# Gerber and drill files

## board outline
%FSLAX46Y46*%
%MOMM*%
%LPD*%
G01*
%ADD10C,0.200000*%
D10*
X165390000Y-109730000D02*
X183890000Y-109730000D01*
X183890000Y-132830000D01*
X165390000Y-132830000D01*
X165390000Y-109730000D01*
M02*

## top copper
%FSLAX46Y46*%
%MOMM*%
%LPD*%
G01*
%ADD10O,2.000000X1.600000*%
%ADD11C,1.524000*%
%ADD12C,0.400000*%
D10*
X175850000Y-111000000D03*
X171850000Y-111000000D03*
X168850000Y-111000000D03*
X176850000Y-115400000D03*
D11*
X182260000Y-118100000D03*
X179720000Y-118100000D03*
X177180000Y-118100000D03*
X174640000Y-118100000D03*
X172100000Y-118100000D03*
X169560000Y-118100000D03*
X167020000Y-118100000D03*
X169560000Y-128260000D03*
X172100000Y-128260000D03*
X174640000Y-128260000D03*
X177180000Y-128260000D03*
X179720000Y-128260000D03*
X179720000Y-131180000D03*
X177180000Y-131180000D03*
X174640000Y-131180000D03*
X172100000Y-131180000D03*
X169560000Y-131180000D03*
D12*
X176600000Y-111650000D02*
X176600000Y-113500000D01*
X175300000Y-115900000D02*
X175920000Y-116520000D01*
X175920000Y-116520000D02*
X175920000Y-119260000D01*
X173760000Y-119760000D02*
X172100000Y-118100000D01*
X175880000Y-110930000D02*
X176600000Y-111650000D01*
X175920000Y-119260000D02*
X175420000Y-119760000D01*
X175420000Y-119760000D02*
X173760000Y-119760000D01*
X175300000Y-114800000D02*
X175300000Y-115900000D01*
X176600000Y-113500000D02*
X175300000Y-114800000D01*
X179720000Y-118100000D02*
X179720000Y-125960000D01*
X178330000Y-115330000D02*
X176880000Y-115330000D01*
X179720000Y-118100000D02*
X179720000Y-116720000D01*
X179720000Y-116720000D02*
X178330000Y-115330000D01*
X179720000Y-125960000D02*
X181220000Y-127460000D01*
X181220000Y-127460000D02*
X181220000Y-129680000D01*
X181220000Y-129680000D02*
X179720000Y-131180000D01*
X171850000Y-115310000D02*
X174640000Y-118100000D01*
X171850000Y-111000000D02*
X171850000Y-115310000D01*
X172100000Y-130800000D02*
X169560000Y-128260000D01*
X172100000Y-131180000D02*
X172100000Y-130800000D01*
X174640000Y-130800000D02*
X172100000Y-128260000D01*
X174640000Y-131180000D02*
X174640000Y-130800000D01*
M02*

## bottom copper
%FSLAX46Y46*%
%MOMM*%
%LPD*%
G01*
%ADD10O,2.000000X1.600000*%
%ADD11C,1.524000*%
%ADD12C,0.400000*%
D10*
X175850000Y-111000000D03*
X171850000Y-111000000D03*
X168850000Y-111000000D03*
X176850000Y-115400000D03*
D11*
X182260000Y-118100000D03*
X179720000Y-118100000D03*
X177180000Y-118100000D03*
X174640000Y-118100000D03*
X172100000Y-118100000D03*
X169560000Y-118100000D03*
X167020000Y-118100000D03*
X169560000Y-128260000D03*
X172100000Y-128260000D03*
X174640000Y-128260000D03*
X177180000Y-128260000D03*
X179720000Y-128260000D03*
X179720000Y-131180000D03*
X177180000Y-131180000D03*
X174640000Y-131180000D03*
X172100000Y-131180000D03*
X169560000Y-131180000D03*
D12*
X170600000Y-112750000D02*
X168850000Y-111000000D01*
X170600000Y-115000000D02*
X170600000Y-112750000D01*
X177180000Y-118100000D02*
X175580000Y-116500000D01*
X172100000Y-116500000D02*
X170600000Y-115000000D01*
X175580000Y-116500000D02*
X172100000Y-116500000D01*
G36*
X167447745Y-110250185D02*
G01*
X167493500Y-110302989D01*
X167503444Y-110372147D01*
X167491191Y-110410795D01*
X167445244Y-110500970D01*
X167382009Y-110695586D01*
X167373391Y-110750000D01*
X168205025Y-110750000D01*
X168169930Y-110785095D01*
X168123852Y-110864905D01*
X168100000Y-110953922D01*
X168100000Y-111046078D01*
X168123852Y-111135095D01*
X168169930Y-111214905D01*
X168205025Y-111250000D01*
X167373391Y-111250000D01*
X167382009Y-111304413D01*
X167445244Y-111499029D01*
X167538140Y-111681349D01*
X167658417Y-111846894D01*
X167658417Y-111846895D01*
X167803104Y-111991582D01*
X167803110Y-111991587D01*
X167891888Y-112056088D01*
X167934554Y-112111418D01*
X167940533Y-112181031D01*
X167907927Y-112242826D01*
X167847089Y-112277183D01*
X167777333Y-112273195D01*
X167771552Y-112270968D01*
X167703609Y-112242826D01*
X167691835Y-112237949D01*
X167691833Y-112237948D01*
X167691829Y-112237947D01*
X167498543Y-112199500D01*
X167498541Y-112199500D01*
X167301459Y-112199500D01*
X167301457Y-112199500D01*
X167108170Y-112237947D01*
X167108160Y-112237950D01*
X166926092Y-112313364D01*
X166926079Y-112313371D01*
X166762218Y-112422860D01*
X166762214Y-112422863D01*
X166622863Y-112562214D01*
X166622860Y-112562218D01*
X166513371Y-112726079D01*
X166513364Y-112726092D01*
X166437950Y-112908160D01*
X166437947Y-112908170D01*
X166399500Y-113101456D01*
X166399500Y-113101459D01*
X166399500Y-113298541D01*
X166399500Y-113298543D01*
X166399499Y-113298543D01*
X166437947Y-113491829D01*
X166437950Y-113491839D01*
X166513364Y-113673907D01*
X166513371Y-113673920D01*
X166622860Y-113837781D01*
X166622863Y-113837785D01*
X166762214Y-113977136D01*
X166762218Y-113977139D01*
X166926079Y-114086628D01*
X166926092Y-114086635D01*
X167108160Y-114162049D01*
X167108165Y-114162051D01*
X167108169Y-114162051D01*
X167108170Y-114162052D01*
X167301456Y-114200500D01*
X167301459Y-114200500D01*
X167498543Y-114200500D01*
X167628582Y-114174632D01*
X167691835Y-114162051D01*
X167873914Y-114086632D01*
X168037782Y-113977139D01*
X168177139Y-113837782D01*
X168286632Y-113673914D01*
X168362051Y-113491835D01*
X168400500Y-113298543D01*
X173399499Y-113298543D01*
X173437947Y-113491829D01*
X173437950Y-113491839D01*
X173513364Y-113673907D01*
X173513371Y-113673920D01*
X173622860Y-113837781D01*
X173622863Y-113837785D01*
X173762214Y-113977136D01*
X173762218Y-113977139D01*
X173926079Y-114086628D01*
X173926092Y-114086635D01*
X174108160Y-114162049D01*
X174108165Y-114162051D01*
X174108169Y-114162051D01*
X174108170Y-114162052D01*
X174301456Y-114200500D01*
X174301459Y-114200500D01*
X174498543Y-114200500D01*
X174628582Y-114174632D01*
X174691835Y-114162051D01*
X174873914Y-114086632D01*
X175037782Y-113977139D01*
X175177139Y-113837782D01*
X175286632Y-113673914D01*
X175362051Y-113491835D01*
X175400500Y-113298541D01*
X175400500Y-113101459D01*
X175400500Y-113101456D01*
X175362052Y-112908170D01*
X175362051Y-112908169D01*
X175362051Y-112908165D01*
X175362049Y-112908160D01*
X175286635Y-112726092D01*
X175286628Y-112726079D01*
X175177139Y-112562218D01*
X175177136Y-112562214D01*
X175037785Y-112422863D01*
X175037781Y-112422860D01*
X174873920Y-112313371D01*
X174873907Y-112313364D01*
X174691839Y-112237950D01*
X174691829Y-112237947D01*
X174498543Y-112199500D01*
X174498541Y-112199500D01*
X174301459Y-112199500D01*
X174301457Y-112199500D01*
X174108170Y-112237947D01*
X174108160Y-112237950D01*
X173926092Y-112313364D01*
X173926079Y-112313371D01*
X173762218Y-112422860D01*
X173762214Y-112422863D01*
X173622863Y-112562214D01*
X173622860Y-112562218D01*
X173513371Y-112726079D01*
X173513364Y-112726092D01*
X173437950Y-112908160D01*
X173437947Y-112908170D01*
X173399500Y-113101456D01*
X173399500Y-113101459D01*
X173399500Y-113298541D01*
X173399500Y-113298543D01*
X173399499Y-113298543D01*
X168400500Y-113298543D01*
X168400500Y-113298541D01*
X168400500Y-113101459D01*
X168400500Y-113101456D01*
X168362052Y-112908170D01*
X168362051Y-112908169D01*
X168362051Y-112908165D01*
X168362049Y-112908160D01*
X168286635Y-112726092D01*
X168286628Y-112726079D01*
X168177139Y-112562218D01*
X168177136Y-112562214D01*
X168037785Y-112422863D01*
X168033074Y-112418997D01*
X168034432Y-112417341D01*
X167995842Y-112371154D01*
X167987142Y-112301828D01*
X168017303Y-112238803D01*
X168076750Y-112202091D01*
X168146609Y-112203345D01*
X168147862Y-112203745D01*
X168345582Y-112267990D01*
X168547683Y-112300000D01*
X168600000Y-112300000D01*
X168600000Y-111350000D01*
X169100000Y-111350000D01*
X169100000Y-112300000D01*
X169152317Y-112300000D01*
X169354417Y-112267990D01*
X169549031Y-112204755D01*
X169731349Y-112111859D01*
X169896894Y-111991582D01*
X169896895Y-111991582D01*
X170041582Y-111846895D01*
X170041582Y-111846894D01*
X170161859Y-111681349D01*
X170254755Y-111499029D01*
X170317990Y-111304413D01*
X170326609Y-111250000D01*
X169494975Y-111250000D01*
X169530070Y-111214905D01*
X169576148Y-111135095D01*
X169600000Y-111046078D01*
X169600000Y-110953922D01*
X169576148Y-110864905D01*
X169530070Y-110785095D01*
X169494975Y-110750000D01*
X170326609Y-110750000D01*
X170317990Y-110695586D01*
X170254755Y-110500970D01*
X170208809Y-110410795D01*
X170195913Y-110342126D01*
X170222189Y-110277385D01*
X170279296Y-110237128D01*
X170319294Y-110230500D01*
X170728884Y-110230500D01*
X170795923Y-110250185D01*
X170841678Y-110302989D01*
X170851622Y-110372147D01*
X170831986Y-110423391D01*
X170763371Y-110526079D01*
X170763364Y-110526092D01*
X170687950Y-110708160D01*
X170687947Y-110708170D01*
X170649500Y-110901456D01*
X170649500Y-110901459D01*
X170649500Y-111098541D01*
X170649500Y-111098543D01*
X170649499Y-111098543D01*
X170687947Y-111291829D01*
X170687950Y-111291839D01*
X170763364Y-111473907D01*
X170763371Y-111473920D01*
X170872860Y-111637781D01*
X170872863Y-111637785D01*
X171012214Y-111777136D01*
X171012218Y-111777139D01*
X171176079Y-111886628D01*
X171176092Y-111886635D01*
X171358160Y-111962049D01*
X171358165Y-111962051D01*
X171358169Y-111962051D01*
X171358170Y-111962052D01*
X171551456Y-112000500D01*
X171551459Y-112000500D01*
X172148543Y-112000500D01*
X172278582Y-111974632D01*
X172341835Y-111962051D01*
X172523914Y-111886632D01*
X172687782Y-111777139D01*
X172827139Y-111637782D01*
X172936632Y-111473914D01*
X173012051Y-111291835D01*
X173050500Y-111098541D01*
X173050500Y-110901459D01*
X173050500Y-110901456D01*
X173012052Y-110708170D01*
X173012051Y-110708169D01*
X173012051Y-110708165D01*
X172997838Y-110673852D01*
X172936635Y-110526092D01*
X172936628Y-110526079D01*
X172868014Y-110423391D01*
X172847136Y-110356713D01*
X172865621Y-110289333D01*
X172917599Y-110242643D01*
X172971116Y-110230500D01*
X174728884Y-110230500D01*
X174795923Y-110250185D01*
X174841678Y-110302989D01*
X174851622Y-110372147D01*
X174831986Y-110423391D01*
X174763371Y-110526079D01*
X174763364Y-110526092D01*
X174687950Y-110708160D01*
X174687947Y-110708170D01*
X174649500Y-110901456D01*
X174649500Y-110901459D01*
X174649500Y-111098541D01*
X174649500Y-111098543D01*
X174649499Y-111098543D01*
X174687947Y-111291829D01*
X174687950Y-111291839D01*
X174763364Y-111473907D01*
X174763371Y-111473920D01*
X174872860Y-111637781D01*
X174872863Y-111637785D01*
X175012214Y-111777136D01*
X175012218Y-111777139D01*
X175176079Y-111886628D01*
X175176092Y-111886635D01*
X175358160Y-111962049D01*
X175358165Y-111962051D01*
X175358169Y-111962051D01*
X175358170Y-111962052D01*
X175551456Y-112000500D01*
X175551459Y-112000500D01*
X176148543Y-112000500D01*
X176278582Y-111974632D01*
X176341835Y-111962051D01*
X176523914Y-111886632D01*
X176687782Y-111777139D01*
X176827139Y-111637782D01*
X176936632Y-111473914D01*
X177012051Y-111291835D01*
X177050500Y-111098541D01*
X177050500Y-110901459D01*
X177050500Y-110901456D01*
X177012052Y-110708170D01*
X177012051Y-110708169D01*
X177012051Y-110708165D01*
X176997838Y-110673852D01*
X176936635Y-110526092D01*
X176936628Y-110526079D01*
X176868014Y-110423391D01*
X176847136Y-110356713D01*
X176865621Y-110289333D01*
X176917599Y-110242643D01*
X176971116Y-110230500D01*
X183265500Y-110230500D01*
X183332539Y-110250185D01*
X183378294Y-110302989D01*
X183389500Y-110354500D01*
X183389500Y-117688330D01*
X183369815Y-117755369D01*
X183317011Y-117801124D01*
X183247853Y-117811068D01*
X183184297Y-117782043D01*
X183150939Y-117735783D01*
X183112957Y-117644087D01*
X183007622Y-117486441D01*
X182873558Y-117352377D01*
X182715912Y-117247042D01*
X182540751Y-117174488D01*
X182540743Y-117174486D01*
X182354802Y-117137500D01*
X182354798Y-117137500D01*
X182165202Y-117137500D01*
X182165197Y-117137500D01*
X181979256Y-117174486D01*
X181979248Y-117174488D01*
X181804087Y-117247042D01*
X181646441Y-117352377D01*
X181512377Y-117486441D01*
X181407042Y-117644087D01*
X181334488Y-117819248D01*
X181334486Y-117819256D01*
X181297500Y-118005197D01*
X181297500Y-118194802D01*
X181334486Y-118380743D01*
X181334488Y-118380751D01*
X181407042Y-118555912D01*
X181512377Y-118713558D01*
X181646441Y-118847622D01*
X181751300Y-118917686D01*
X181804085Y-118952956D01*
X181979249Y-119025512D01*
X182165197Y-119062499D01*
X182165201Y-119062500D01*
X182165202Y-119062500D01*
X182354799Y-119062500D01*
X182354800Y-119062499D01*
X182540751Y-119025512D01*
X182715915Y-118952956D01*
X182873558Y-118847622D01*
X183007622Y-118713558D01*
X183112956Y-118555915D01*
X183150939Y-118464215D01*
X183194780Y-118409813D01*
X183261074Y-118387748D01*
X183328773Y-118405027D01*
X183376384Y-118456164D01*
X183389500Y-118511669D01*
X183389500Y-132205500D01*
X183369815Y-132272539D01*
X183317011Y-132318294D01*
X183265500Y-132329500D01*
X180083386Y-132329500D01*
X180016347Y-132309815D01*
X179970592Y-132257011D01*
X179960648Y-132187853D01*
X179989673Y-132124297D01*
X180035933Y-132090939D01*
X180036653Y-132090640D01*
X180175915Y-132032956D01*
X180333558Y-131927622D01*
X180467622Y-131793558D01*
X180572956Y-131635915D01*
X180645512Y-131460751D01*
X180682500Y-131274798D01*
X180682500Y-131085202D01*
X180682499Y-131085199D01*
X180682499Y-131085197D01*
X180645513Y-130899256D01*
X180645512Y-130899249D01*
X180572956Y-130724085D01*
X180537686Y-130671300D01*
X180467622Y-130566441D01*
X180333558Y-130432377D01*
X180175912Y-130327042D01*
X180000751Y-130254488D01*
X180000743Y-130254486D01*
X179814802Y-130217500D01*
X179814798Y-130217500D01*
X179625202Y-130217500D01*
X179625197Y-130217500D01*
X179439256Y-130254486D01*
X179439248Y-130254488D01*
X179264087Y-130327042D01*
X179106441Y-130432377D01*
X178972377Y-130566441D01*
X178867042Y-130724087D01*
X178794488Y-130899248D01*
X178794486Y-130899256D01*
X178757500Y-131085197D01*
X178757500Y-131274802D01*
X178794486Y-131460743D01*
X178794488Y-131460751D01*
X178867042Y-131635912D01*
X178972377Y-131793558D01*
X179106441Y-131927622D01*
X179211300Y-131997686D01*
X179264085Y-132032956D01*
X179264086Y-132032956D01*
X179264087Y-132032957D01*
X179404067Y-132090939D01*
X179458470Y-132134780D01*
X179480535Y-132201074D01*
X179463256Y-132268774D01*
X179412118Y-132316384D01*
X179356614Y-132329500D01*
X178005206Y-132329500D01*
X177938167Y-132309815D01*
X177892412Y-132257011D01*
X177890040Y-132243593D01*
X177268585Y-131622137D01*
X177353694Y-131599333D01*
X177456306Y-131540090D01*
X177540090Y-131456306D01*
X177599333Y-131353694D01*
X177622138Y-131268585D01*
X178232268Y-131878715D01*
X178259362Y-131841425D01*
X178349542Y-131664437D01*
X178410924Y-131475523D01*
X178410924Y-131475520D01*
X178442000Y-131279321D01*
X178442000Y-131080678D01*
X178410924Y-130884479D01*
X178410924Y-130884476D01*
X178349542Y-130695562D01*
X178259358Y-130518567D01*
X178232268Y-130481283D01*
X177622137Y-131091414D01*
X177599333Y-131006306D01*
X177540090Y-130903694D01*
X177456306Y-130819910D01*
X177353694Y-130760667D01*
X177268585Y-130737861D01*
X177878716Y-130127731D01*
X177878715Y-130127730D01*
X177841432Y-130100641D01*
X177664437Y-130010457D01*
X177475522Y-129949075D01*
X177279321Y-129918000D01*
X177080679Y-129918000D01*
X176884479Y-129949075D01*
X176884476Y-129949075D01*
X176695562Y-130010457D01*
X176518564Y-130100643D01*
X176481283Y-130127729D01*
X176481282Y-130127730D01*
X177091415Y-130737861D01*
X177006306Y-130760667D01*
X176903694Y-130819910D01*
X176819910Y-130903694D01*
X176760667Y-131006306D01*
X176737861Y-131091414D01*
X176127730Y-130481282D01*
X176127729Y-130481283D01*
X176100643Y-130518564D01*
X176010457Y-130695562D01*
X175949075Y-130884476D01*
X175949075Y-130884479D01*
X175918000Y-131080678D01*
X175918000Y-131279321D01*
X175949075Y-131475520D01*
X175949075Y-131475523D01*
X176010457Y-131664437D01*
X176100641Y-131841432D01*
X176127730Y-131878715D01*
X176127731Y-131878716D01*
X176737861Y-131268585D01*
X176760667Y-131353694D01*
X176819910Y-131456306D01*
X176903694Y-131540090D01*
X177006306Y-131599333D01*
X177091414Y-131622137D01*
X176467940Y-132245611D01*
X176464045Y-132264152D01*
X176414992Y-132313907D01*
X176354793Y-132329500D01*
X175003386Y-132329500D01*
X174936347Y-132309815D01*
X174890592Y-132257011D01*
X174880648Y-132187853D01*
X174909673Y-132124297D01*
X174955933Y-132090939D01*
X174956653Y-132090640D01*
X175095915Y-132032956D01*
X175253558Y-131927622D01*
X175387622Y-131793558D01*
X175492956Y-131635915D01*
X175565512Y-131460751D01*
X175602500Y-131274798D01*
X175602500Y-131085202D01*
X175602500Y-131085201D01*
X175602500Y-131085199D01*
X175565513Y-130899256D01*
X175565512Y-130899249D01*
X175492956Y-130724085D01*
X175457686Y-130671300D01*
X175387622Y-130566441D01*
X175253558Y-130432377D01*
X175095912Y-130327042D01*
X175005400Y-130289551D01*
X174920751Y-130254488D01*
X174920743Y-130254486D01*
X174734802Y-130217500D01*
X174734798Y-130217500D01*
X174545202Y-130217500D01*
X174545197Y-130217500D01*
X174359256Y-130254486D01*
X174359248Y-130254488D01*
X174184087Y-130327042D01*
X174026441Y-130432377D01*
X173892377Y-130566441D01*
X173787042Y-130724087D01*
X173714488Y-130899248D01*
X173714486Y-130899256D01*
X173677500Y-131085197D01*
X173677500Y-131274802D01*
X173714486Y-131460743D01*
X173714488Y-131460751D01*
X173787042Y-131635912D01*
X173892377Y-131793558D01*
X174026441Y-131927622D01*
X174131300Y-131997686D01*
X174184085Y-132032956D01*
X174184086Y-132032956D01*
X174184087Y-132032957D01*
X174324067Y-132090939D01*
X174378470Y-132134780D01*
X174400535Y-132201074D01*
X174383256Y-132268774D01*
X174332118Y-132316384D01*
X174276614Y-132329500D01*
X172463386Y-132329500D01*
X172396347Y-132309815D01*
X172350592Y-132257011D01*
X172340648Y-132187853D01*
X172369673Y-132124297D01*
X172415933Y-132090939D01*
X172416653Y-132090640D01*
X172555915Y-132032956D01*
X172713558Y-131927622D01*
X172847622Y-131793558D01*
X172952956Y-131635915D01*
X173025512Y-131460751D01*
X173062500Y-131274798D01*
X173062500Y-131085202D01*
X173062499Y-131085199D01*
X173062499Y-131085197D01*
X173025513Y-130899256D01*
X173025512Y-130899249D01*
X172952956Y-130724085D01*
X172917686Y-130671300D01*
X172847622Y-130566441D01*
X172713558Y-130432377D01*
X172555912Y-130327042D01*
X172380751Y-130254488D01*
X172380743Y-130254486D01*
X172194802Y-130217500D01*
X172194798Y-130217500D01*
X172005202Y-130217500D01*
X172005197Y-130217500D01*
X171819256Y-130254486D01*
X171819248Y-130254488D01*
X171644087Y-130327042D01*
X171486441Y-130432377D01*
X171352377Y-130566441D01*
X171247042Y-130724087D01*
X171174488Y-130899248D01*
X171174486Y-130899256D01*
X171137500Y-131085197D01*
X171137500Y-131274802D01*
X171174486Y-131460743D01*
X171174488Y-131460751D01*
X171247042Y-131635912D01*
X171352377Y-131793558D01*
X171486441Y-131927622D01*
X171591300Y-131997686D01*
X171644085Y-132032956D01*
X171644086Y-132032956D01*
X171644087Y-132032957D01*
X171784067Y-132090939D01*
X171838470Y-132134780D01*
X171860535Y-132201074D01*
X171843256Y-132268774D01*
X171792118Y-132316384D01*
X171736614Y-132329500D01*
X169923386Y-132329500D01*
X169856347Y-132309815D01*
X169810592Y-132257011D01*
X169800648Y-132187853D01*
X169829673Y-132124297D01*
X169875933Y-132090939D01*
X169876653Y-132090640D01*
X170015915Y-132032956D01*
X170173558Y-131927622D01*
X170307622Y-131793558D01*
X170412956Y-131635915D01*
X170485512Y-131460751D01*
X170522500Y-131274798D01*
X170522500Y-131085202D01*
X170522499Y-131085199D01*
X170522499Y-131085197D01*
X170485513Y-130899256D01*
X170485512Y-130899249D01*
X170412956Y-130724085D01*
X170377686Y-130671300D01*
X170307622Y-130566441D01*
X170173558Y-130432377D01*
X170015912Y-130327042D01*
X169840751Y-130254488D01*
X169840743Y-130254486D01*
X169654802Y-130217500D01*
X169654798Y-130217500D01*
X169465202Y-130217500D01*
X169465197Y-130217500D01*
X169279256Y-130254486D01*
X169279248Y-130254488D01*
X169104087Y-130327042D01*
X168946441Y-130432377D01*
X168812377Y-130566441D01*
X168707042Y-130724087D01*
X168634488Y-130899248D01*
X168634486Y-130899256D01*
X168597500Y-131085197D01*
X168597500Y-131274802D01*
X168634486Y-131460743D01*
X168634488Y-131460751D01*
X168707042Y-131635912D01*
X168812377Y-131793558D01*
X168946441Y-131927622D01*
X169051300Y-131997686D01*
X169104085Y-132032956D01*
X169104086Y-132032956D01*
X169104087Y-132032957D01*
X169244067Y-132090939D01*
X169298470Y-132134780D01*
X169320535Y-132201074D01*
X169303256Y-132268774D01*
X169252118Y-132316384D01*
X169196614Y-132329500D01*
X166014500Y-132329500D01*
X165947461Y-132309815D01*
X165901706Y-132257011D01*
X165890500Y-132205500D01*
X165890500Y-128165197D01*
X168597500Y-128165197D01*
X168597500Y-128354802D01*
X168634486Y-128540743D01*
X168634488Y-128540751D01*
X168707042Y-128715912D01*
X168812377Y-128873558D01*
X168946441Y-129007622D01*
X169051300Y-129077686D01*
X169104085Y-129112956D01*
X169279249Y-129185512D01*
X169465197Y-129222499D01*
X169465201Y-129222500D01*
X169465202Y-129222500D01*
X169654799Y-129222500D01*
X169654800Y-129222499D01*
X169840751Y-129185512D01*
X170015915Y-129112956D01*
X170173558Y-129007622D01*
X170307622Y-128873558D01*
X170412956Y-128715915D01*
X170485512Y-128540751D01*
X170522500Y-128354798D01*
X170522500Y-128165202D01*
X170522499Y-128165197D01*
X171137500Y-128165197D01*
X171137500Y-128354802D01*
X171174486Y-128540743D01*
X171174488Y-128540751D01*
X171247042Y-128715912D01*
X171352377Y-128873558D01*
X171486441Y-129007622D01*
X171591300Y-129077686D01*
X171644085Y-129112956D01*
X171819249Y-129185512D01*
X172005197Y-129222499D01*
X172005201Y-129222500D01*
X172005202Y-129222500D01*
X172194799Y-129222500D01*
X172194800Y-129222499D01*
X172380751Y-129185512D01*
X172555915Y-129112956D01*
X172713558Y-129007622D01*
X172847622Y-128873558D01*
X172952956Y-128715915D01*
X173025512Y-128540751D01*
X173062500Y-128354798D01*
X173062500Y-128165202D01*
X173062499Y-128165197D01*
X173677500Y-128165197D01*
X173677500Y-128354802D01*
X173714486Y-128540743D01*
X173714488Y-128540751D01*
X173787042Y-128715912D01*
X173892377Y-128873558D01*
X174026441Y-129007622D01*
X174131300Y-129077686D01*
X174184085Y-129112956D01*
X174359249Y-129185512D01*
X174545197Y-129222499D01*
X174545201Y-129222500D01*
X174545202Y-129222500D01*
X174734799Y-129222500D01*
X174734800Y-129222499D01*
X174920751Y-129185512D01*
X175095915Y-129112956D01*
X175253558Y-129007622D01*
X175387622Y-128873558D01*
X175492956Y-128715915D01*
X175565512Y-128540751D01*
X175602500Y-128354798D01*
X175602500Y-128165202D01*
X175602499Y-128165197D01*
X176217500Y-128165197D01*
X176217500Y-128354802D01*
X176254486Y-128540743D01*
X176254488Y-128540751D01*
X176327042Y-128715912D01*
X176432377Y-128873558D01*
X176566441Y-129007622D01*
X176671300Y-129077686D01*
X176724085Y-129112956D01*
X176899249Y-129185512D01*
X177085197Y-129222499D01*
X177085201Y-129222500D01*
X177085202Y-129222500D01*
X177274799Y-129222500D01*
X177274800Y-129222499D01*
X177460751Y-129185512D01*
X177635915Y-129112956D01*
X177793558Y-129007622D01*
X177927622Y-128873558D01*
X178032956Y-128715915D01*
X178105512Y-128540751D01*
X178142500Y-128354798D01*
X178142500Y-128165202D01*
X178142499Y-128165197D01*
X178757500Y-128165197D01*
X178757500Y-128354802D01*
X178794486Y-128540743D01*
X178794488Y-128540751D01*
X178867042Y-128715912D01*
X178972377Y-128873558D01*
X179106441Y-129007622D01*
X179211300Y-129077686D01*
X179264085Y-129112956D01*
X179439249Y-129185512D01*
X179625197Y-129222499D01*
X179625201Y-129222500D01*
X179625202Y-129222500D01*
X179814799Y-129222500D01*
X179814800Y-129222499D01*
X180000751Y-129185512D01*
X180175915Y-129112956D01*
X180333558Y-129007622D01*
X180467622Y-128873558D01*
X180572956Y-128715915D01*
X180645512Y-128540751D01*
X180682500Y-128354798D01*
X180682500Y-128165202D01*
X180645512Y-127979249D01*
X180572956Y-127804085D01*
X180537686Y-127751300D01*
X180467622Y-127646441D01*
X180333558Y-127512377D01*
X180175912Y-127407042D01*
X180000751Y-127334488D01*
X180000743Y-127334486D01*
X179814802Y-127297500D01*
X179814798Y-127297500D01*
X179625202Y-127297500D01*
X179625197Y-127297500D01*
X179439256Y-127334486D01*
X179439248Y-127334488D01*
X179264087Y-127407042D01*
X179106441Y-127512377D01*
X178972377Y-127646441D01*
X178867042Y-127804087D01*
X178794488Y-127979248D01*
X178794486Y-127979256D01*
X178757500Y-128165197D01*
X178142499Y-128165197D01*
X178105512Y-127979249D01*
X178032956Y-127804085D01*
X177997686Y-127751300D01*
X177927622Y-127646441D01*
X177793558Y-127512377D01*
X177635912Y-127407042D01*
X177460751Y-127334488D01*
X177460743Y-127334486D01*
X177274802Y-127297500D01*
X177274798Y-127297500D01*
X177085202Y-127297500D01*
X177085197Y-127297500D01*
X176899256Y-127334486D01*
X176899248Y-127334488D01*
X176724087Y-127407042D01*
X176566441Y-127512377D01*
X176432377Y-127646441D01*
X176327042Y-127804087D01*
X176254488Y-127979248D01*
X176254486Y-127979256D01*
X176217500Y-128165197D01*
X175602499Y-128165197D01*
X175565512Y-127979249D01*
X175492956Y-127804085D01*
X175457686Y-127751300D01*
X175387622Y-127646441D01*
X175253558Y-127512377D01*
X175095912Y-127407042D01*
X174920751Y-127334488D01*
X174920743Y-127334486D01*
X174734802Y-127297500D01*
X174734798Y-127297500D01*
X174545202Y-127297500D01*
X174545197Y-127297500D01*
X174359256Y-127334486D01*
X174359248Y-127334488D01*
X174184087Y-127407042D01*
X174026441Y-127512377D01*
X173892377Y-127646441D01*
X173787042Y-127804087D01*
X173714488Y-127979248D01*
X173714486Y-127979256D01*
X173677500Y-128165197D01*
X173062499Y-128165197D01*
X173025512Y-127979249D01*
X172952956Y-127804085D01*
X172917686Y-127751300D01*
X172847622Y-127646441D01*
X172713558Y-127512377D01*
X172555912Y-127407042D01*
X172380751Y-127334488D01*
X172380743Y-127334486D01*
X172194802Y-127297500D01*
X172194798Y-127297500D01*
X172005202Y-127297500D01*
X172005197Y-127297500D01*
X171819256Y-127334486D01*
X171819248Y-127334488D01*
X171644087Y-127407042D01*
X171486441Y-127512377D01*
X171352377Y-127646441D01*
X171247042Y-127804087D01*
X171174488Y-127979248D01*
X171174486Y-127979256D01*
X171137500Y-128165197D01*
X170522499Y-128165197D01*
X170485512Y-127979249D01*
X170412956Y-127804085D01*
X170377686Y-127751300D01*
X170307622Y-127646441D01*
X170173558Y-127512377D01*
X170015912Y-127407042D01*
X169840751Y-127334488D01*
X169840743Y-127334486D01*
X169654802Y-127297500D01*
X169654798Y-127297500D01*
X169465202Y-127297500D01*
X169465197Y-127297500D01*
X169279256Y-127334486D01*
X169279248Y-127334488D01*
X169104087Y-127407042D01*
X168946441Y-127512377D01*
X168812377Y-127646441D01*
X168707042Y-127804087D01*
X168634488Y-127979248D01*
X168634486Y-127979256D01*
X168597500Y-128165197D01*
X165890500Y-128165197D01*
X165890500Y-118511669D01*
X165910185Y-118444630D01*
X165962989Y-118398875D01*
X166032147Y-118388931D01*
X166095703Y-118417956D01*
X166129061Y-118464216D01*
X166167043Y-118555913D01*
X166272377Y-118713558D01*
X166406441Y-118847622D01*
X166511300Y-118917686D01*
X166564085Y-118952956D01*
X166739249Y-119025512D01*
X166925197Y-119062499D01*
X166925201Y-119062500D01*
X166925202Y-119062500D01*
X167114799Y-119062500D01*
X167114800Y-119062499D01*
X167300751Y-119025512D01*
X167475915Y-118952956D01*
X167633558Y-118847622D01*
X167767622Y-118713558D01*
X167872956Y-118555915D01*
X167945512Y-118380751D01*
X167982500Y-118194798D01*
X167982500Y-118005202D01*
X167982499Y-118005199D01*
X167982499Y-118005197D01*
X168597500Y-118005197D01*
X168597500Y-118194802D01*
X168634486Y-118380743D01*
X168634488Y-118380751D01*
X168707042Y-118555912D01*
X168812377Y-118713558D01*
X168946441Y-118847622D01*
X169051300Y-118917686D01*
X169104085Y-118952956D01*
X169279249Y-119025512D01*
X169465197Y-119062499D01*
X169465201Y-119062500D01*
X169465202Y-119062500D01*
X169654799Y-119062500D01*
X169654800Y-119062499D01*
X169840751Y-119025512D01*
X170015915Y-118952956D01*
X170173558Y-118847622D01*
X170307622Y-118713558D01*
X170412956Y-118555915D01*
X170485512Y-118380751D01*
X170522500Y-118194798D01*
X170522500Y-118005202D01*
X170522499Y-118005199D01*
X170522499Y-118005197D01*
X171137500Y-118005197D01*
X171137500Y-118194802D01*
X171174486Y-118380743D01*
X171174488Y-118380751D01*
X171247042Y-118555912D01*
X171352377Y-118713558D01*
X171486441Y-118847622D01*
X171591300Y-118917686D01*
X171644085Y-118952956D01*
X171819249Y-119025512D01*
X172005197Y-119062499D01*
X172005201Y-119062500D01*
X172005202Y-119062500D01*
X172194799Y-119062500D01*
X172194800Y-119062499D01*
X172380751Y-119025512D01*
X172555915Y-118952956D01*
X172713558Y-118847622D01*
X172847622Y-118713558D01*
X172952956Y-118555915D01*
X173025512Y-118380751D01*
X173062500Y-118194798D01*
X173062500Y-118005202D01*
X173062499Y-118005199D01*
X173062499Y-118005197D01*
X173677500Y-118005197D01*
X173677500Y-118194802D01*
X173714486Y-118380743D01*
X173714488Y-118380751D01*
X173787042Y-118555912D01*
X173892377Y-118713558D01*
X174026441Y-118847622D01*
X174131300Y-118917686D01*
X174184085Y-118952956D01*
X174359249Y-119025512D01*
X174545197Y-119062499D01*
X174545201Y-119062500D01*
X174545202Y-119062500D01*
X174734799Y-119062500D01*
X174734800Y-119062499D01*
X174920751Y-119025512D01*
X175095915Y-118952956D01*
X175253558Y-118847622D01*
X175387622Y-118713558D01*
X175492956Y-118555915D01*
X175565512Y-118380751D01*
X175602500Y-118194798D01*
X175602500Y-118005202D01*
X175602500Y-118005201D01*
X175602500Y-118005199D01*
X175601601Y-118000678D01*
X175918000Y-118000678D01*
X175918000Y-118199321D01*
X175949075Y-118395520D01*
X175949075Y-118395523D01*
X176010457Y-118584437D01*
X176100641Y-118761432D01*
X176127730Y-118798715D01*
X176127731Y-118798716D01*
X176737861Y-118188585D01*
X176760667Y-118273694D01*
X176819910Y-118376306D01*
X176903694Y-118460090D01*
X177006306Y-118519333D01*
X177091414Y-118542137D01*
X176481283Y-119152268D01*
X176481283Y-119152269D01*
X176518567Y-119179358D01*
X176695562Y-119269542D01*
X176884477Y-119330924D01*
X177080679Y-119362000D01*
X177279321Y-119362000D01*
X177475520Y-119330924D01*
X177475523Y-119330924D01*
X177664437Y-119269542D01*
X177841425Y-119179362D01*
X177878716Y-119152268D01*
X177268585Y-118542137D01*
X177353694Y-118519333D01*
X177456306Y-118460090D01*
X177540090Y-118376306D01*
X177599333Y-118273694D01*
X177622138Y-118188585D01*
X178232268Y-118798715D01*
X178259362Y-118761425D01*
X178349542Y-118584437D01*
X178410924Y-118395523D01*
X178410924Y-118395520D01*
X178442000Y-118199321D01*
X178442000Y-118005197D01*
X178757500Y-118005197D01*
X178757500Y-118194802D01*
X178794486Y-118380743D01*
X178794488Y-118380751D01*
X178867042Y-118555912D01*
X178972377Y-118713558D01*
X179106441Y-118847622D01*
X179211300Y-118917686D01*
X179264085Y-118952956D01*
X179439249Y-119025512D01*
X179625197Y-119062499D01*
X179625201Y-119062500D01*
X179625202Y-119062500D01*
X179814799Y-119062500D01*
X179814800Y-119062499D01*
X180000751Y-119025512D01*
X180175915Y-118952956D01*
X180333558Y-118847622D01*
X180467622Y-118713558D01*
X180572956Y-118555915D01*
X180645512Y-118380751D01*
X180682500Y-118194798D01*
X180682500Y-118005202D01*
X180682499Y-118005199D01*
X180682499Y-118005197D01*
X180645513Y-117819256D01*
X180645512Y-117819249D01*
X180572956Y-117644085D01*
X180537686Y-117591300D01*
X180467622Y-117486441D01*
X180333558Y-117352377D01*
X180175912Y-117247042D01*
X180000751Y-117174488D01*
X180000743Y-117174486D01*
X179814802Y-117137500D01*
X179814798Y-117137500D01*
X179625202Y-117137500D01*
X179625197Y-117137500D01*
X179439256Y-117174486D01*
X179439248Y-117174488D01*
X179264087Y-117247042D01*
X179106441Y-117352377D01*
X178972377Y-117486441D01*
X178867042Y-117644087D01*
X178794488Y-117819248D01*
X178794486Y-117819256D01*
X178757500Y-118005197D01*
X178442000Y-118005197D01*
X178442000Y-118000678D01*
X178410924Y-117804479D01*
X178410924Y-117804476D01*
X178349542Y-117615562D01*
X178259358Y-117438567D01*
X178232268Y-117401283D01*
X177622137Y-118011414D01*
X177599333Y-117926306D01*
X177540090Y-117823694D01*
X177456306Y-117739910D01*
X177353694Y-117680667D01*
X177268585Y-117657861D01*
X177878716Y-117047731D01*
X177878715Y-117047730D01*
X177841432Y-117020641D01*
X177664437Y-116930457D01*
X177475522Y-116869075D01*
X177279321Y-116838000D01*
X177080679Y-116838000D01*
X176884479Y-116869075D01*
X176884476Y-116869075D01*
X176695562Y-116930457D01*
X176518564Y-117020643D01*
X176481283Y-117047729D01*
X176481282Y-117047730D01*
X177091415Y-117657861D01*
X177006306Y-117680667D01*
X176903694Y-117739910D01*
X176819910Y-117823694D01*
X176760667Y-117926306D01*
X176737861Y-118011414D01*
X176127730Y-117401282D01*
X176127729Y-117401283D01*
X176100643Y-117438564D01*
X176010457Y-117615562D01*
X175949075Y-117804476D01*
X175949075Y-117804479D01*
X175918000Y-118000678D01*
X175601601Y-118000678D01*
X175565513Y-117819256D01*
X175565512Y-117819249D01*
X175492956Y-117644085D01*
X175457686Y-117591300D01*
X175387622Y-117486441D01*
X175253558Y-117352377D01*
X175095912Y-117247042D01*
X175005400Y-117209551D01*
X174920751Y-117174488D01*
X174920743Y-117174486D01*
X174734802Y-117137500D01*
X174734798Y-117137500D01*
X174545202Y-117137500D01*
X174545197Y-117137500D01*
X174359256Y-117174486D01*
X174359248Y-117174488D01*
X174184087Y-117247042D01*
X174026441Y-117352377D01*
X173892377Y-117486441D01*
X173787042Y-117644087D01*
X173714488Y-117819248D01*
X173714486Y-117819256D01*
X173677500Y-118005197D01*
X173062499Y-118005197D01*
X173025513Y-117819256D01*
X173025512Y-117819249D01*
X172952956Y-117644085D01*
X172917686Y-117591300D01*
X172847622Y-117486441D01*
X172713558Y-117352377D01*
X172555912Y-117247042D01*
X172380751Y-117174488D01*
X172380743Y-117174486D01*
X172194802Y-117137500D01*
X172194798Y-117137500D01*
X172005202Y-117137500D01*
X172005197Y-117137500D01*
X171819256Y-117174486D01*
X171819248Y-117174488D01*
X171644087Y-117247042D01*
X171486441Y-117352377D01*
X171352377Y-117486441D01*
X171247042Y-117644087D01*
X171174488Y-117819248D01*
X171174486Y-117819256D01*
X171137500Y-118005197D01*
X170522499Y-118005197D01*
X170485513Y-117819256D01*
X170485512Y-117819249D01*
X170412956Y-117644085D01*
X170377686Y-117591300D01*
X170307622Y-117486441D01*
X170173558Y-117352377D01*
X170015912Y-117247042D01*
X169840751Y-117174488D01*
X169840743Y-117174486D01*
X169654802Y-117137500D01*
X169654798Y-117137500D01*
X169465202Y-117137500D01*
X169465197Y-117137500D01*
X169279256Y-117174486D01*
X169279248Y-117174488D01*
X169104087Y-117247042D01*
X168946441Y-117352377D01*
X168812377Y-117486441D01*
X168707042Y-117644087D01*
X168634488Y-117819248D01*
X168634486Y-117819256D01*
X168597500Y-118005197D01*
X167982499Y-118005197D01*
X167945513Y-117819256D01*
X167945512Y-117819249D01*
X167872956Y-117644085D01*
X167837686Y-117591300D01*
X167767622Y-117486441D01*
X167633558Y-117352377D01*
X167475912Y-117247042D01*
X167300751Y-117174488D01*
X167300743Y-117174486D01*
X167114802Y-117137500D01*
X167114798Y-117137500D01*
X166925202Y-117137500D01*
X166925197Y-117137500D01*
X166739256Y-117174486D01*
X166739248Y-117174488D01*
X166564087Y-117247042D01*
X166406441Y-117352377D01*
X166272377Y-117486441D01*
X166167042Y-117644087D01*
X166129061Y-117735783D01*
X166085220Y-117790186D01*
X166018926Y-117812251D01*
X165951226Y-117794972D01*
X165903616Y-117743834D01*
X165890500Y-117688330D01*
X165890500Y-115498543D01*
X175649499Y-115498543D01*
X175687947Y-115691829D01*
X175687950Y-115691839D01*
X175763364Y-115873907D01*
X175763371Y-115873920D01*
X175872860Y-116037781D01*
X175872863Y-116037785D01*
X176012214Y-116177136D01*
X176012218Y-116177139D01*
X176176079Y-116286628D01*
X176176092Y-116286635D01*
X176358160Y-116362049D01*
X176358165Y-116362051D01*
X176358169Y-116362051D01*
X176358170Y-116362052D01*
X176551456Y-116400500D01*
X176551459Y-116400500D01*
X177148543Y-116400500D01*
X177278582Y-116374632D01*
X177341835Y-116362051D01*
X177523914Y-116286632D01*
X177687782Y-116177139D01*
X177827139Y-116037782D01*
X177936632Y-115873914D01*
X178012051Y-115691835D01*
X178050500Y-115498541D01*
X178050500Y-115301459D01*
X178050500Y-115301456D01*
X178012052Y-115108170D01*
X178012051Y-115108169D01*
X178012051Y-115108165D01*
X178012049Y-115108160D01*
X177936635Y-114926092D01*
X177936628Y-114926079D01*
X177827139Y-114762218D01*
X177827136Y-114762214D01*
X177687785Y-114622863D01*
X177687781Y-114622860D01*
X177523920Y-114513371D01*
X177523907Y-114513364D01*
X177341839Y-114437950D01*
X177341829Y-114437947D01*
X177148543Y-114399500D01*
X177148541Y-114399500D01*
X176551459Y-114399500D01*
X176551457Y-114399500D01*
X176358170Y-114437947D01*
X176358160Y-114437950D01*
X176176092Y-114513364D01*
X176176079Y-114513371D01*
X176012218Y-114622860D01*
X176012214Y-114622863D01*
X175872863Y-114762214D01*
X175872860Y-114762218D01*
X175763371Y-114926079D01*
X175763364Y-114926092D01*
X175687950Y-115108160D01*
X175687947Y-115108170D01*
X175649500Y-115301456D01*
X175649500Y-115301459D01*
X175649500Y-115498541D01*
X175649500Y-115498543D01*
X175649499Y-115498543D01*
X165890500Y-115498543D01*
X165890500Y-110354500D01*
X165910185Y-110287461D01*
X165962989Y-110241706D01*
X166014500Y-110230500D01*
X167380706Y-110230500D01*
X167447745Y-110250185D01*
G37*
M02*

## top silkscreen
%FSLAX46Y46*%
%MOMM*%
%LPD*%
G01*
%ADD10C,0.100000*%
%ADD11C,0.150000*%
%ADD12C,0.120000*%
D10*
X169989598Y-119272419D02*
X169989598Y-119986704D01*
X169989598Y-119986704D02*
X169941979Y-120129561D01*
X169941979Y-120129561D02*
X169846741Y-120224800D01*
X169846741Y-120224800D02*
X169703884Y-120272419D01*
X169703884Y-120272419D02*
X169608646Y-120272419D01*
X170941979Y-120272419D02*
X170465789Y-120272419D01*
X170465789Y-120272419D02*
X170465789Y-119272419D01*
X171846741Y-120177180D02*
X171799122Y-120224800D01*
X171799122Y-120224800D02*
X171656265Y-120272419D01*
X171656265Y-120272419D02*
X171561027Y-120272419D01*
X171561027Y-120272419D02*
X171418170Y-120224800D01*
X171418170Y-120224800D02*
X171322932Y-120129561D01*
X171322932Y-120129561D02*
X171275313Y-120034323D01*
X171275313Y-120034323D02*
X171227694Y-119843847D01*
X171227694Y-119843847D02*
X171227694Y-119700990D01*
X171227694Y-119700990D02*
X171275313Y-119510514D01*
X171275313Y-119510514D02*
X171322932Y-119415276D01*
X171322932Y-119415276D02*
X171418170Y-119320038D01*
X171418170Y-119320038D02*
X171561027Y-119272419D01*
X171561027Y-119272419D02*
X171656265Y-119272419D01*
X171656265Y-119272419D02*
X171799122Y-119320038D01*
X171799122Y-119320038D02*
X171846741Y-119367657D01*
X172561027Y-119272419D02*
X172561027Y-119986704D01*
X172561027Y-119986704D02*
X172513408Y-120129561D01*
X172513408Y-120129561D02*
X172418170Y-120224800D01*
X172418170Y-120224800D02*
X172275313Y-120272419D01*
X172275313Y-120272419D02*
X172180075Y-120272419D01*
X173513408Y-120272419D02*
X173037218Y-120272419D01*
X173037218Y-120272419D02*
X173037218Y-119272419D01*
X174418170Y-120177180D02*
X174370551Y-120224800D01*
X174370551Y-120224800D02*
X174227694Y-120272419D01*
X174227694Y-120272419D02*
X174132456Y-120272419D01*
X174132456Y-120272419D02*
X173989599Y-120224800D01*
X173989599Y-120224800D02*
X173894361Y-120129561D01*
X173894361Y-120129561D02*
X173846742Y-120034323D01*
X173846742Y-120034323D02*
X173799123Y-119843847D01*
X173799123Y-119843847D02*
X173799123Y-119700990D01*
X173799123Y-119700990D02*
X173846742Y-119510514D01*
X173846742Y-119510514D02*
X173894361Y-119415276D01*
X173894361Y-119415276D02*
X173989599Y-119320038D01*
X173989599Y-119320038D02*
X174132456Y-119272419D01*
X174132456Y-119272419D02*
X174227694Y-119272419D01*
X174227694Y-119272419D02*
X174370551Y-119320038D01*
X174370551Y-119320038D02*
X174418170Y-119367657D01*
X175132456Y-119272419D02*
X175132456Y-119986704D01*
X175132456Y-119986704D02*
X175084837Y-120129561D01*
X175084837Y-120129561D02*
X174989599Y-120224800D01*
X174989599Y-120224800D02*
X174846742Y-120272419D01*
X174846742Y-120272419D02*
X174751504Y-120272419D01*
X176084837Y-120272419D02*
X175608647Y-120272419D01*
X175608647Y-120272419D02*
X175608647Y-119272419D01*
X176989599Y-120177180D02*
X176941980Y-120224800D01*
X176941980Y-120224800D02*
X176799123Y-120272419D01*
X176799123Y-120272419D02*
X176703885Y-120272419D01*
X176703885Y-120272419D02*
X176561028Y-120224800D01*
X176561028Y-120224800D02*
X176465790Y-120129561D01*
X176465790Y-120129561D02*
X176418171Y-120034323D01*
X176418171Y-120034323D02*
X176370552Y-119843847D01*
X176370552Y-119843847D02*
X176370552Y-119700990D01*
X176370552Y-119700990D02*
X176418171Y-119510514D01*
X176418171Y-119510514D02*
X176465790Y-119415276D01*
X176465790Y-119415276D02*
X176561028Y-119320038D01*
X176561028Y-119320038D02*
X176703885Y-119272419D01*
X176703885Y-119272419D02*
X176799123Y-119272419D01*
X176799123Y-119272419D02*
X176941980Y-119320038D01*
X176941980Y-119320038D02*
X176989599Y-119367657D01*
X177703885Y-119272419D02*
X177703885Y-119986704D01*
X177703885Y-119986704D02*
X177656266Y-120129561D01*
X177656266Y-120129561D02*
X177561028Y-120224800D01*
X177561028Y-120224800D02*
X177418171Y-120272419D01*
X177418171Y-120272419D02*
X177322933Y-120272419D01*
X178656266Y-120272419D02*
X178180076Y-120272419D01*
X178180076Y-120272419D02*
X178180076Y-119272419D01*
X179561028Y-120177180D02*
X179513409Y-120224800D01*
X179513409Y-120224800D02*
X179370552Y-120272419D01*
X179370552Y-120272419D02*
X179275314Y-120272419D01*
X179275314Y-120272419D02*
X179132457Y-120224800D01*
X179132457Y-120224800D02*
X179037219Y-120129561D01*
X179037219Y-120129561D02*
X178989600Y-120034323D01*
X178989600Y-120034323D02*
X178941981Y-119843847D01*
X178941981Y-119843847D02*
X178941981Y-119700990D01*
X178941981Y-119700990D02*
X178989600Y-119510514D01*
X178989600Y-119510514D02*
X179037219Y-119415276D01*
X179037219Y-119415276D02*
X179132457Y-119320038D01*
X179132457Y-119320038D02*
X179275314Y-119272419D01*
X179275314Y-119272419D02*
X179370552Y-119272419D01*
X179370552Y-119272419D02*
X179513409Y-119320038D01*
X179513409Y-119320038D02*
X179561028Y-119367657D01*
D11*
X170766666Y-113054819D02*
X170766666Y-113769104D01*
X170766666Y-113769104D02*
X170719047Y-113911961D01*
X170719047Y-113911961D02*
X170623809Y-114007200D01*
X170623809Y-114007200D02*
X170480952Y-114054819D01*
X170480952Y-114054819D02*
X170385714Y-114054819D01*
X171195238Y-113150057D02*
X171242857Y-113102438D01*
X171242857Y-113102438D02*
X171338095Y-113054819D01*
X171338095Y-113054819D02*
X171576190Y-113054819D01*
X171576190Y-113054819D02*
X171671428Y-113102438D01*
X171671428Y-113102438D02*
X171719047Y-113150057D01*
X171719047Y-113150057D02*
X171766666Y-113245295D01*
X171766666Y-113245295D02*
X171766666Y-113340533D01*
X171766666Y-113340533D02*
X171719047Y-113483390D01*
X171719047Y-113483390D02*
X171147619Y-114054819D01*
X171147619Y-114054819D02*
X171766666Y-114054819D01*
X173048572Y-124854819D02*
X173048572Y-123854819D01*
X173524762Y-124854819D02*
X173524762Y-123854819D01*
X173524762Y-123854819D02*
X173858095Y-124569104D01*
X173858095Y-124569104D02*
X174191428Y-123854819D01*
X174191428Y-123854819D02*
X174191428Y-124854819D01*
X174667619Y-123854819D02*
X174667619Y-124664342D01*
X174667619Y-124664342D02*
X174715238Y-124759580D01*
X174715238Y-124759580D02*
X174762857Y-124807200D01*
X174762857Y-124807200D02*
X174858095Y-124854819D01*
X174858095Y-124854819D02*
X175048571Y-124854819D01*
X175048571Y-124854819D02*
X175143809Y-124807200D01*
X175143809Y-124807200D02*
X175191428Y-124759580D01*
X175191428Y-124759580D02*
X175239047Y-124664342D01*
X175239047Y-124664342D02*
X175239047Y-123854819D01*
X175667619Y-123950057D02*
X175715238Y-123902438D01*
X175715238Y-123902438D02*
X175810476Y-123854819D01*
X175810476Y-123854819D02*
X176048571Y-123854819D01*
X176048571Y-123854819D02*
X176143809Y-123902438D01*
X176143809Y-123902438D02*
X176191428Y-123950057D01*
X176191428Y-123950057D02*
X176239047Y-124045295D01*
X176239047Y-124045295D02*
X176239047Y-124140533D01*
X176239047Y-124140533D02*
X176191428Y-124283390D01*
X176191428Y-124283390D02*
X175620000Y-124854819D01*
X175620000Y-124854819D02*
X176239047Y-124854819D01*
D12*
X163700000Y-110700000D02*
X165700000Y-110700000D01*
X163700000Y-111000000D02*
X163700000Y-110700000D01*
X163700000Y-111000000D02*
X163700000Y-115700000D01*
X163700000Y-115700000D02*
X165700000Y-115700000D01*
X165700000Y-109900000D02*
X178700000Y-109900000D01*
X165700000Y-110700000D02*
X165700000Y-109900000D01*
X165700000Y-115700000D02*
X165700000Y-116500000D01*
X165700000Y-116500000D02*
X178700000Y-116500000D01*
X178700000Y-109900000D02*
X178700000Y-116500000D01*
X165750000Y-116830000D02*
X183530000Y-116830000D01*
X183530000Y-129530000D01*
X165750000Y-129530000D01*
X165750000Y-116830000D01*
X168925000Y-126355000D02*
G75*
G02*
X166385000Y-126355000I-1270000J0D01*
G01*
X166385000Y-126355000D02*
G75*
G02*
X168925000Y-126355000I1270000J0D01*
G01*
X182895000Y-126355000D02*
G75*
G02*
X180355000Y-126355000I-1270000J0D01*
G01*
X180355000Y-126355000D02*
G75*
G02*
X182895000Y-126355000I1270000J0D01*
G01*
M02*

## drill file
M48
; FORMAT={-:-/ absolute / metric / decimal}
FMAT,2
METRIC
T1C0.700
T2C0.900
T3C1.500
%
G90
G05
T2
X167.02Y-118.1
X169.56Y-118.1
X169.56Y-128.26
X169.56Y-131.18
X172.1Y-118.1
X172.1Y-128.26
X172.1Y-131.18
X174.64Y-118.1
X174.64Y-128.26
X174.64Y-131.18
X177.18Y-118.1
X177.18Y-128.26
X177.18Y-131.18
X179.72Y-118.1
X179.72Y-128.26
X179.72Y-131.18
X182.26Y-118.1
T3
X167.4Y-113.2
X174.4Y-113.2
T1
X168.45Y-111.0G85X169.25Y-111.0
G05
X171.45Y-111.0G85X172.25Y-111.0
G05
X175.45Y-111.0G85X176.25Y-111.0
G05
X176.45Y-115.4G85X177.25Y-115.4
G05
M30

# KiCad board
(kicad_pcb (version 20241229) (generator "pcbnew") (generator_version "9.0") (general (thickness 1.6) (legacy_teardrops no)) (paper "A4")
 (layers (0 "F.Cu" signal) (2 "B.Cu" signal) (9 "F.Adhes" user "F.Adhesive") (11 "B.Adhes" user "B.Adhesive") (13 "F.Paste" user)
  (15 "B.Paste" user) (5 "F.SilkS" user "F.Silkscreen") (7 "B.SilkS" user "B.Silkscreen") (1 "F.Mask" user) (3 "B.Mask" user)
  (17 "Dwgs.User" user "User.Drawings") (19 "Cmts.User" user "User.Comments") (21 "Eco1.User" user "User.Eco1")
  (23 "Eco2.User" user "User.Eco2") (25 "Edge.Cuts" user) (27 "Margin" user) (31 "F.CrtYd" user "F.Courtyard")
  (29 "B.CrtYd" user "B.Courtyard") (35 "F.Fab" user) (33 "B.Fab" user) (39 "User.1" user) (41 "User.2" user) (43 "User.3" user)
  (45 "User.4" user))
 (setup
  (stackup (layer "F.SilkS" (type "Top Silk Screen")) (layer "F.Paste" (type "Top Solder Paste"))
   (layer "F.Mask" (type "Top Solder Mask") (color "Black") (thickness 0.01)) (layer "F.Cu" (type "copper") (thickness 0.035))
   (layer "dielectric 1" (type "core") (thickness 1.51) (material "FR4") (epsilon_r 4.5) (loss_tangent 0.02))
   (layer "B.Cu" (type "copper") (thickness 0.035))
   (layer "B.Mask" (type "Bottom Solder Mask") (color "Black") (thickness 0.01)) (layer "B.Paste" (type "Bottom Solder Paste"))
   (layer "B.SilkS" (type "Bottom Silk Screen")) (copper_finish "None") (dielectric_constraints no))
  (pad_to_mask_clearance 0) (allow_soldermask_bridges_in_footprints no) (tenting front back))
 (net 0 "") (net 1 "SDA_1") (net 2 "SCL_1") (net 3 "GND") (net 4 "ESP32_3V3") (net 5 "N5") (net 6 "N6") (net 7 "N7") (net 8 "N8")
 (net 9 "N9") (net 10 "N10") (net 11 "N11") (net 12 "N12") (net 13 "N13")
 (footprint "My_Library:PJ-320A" (layer "F.Cu") (at 163.7 111)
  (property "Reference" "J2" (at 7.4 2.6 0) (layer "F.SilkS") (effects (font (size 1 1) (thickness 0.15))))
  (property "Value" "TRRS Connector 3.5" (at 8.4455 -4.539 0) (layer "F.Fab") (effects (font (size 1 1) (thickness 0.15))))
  (fp_line (start 0 -0.3) (end 2 -0.3) (stroke (width 0.12) (type solid)) (layer "F.SilkS"))
  (fp_line (start 0 0) (end 0 -0.3) (stroke (width 0.12) (type solid)) (layer "F.SilkS"))
  (fp_line (start 0 0) (end 0 4.7) (stroke (width 0.12) (type solid)) (layer "F.SilkS"))
  (fp_line (start 0 4.7) (end 2 4.7) (stroke (width 0.12) (type solid)) (layer "F.SilkS"))
  (fp_line (start 2 -1.1) (end 15 -1.1) (stroke (width 0.12) (type solid)) (layer "F.SilkS"))
  (fp_line (start 2 -0.3) (end 2 -1.1) (stroke (width 0.12) (type solid)) (layer "F.SilkS"))
  (fp_line (start 2 4.7) (end 2 5.5) (stroke (width 0.12) (type solid)) (layer "F.SilkS"))
  (fp_line (start 2 5.5) (end 15 5.5) (stroke (width 0.12) (type solid)) (layer "F.SilkS"))
  (fp_line (start 15 -1.1) (end 15 5.5) (stroke (width 0.12) (type solid)) (layer "F.SilkS"))
  (pad "" np_thru_hole circle (at 3.7 2.2) (size 1.5 1.5) (drill 1.5) (layers "*.Cu"))
  (pad "" np_thru_hole circle (at 10.7 2.2) (size 1.5 1.5) (drill 1.5) (layers "*.Cu"))
  (pad "R1" thru_hole oval (at 12.15 0) (size 2 1.6) (drill oval 1.5 0.7) (layers "*.Cu" "*.Mask") (remove_unused_layers no) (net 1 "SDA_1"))
  (pad "R2" thru_hole oval (at 8.15 0) (size 2 1.6) (drill oval 1.5 0.7) (layers "*.Cu" "*.Mask") (remove_unused_layers no) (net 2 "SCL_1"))
  (pad "S" thru_hole oval (at 5.15 0) (size 2 1.6) (drill oval 1.5 0.7) (layers "*.Cu" "*.Mask") (remove_unused_layers no) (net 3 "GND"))
  (pad "T" thru_hole oval (at 13.15 4.4) (size 2 1.6) (drill oval 1.5 0.7) (layers "*.Cu" "*.Mask") (remove_unused_layers no)
   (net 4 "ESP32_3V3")))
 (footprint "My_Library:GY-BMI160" (layer "F.Cu") (at 174.64 123.18 -90)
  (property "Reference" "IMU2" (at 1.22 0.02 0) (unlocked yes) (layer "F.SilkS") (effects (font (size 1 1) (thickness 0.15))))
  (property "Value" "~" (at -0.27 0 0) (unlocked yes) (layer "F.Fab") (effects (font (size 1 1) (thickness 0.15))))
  (fp_rect (start -6.35 -8.89) (end 6.35 8.89) (stroke (width 0.12) (type default)) (fill no) (layer "F.SilkS"))
  (fp_circle (center 3.175 6.985) (end 1.905 6.985) (stroke (width 0.12) (type default)) (fill no) (layer "F.SilkS"))
  (fp_circle (center 3.175 -6.985) (end 1.905 -6.985) (stroke (width 0.12) (type default)) (fill no) (layer "F.SilkS"))
  (pad "1" thru_hole circle (at -5.08 -7.62 270) (size 1.524 1.524) (drill 0.9) (layers "*.Cu" "*.Mask") (remove_unused_layers no)
   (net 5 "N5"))
  (pad "2" thru_hole circle (at -5.08 -5.08 270) (size 1.524 1.524) (drill 0.9) (layers "*.Cu" "*.Mask") (remove_unused_layers no)
   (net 4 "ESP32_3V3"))
  (pad "3" thru_hole circle (at -5.08 -2.54 270) (size 1.524 1.524) (drill 0.9) (layers "*.Cu" "*.Mask") (remove_unused_layers no)
   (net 3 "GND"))
  (pad "4" thru_hole circle (at -5.08 0 270) (size 1.524 1.524) (drill 0.9) (layers "*.Cu" "*.Mask") (remove_unused_layers no)
   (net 2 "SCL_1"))
  (pad "5" thru_hole circle (at -5.08 2.54 270) (size 1.524 1.524) (drill 0.9) (layers "*.Cu" "*.Mask") (remove_unused_layers no)
   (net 1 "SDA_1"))
  (pad "6" thru_hole circle (at -5.08 5.08 270) (size 1.524 1.524) (drill 0.9) (layers "*.Cu" "*.Mask") (remove_unused_layers no)
   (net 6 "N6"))
  (pad "7" thru_hole circle (at -5.08 7.62 270) (size 1.524 1.524) (drill 0.9) (layers "*.Cu" "*.Mask") (remove_unused_layers no)
   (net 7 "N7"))
  (pad "8" thru_hole circle (at 5.08 5.08 270) (size 1.524 1.524) (drill 0.9) (layers "*.Cu" "*.Mask") (remove_unused_layers no)
   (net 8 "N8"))
  (pad "9" thru_hole circle (at 5.08 2.54 270) (size 1.524 1.524) (drill 0.9) (layers "*.Cu" "*.Mask") (remove_unused_layers no)
   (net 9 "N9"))
  (pad "10" thru_hole circle (at 5.08 0 270) (size 1.524 1.524) (drill 0.9) (layers "*.Cu" "*.Mask") (remove_unused_layers no)
   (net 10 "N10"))
  (pad "11" thru_hole circle (at 5.08 -2.54 270) (size 1.524 1.524) (drill 0.9) (layers "*.Cu" "*.Mask") (remove_unused_layers no)
   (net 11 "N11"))
  (pad "12" thru_hole circle (at 5.08 -5.08 270) (size 1.524 1.524) (drill 0.9) (layers "*.Cu" "*.Mask") (remove_unused_layers no)
   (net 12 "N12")))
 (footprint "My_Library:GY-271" (layer "B.Cu") (at 174.64 126.18 90)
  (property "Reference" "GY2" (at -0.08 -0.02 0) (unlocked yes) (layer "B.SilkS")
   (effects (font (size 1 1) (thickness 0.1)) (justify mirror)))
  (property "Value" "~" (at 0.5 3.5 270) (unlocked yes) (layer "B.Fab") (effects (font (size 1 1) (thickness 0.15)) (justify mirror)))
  (pad "1" thru_hole circle (at -5 5.08 90) (size 1.524 1.524) (drill 0.9) (layers "*.Cu" "*.Mask") (remove_unused_layers no)
   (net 4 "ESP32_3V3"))
  (pad "2" thru_hole circle (at -5 2.54 90) (size 1.524 1.524) (drill 0.9) (layers "*.Cu" "*.Mask") (remove_unused_layers no) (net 3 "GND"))
  (pad "3" thru_hole circle (at -5 0 90) (size 1.524 1.524) (drill 0.9) (layers "*.Cu" "*.Mask") (remove_unused_layers no) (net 9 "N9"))
  (pad "4" thru_hole circle (at -5 -2.54 90) (size 1.524 1.524) (drill 0.9) (layers "*.Cu" "*.Mask") (remove_unused_layers no) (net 8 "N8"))
  (pad "5" thru_hole circle (at -5 -5.08 90) (size 1.524 1.524) (drill 0.9) (layers "*.Cu" "*.Mask") (remove_unused_layers no)
   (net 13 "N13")))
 (gr_rect (start 165.39 109.73) (end 183.89 132.83) (stroke (width 0.2) (type solid)) (fill no) (layer "Edge.Cuts"))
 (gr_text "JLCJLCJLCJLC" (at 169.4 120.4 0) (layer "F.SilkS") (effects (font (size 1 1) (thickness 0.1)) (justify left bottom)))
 (segment (start 176.6 111.65) (end 176.6 113.5) (width 0.4) (layer "F.Cu") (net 1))
 (segment (start 175.3 115.9) (end 175.92 116.52) (width 0.4) (layer "F.Cu") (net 1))
 (segment (start 175.92 116.52) (end 175.92 119.26) (width 0.4) (layer "F.Cu") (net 1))
 (segment (start 173.76 119.76) (end 172.1 118.1) (width 0.4) (layer "F.Cu") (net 1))
 (segment (start 175.88 110.93) (end 176.6 111.65) (width 0.4) (layer "F.Cu") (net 1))
 (segment (start 175.92 119.26) (end 175.42 119.76) (width 0.4) (layer "F.Cu") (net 1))
 (segment (start 175.42 119.76) (end 173.76 119.76) (width 0.4) (layer "F.Cu") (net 1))
 (segment (start 175.3 114.8) (end 175.3 115.9) (width 0.4) (layer "F.Cu") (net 1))
 (segment (start 176.6 113.5) (end 175.3 114.8) (width 0.4) (layer "F.Cu") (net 1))
 (segment (start 179.72 118.1) (end 179.72 125.96) (width 0.4) (layer "F.Cu") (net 4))
 (segment (start 178.33 115.33) (end 176.88 115.33) (width 0.4) (layer "F.Cu") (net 4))
 (segment (start 179.72 118.1) (end 179.72 116.72) (width 0.4) (layer "F.Cu") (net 4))
 (segment (start 179.72 116.72) (end 178.33 115.33) (width 0.4) (layer "F.Cu") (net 4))
 (segment (start 179.72 125.96) (end 181.22 127.46) (width 0.4) (layer "F.Cu") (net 4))
 (segment (start 181.22 127.46) (end 181.22 129.68) (width 0.4) (layer "F.Cu") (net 4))
 (segment (start 181.22 129.68) (end 179.72 131.18) (width 0.4) (layer "F.Cu") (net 4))
 (segment (start 171.85 115.31) (end 174.64 118.1) (width 0.4) (layer "F.Cu") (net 2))
 (segment (start 171.85 111) (end 171.85 115.31) (width 0.4) (layer "F.Cu") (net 2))
 (segment (start 170.6 112.75) (end 168.85 111) (width 0.4) (layer "B.Cu") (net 3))
 (segment (start 170.6 115) (end 170.6 112.75) (width 0.4) (layer "B.Cu") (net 3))
 (segment (start 177.18 118.1) (end 175.58 116.5) (width 0.4) (layer "B.Cu") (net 3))
 (segment (start 172.1 116.5) (end 170.6 115) (width 0.4) (layer "B.Cu") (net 3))
 (segment (start 175.58 116.5) (end 172.1 116.5) (width 0.4) (layer "B.Cu") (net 3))
 (segment (start 172.1 130.8) (end 169.56 128.26) (width 0.4) (layer "F.Cu") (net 8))
 (segment (start 172.1 131.18) (end 172.1 130.8) (width 0.4) (layer "F.Cu") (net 8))
 (segment (start 174.64 130.8) (end 172.1 128.26) (width 0.4) (layer "F.Cu") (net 9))
 (segment (start 174.64 131.18) (end 174.64 130.8) (width 0.4) (layer "F.Cu") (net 9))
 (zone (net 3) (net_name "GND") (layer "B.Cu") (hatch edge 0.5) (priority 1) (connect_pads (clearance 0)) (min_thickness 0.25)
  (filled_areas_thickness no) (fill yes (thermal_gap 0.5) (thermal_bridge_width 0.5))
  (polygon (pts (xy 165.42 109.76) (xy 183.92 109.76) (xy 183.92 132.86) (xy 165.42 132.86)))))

